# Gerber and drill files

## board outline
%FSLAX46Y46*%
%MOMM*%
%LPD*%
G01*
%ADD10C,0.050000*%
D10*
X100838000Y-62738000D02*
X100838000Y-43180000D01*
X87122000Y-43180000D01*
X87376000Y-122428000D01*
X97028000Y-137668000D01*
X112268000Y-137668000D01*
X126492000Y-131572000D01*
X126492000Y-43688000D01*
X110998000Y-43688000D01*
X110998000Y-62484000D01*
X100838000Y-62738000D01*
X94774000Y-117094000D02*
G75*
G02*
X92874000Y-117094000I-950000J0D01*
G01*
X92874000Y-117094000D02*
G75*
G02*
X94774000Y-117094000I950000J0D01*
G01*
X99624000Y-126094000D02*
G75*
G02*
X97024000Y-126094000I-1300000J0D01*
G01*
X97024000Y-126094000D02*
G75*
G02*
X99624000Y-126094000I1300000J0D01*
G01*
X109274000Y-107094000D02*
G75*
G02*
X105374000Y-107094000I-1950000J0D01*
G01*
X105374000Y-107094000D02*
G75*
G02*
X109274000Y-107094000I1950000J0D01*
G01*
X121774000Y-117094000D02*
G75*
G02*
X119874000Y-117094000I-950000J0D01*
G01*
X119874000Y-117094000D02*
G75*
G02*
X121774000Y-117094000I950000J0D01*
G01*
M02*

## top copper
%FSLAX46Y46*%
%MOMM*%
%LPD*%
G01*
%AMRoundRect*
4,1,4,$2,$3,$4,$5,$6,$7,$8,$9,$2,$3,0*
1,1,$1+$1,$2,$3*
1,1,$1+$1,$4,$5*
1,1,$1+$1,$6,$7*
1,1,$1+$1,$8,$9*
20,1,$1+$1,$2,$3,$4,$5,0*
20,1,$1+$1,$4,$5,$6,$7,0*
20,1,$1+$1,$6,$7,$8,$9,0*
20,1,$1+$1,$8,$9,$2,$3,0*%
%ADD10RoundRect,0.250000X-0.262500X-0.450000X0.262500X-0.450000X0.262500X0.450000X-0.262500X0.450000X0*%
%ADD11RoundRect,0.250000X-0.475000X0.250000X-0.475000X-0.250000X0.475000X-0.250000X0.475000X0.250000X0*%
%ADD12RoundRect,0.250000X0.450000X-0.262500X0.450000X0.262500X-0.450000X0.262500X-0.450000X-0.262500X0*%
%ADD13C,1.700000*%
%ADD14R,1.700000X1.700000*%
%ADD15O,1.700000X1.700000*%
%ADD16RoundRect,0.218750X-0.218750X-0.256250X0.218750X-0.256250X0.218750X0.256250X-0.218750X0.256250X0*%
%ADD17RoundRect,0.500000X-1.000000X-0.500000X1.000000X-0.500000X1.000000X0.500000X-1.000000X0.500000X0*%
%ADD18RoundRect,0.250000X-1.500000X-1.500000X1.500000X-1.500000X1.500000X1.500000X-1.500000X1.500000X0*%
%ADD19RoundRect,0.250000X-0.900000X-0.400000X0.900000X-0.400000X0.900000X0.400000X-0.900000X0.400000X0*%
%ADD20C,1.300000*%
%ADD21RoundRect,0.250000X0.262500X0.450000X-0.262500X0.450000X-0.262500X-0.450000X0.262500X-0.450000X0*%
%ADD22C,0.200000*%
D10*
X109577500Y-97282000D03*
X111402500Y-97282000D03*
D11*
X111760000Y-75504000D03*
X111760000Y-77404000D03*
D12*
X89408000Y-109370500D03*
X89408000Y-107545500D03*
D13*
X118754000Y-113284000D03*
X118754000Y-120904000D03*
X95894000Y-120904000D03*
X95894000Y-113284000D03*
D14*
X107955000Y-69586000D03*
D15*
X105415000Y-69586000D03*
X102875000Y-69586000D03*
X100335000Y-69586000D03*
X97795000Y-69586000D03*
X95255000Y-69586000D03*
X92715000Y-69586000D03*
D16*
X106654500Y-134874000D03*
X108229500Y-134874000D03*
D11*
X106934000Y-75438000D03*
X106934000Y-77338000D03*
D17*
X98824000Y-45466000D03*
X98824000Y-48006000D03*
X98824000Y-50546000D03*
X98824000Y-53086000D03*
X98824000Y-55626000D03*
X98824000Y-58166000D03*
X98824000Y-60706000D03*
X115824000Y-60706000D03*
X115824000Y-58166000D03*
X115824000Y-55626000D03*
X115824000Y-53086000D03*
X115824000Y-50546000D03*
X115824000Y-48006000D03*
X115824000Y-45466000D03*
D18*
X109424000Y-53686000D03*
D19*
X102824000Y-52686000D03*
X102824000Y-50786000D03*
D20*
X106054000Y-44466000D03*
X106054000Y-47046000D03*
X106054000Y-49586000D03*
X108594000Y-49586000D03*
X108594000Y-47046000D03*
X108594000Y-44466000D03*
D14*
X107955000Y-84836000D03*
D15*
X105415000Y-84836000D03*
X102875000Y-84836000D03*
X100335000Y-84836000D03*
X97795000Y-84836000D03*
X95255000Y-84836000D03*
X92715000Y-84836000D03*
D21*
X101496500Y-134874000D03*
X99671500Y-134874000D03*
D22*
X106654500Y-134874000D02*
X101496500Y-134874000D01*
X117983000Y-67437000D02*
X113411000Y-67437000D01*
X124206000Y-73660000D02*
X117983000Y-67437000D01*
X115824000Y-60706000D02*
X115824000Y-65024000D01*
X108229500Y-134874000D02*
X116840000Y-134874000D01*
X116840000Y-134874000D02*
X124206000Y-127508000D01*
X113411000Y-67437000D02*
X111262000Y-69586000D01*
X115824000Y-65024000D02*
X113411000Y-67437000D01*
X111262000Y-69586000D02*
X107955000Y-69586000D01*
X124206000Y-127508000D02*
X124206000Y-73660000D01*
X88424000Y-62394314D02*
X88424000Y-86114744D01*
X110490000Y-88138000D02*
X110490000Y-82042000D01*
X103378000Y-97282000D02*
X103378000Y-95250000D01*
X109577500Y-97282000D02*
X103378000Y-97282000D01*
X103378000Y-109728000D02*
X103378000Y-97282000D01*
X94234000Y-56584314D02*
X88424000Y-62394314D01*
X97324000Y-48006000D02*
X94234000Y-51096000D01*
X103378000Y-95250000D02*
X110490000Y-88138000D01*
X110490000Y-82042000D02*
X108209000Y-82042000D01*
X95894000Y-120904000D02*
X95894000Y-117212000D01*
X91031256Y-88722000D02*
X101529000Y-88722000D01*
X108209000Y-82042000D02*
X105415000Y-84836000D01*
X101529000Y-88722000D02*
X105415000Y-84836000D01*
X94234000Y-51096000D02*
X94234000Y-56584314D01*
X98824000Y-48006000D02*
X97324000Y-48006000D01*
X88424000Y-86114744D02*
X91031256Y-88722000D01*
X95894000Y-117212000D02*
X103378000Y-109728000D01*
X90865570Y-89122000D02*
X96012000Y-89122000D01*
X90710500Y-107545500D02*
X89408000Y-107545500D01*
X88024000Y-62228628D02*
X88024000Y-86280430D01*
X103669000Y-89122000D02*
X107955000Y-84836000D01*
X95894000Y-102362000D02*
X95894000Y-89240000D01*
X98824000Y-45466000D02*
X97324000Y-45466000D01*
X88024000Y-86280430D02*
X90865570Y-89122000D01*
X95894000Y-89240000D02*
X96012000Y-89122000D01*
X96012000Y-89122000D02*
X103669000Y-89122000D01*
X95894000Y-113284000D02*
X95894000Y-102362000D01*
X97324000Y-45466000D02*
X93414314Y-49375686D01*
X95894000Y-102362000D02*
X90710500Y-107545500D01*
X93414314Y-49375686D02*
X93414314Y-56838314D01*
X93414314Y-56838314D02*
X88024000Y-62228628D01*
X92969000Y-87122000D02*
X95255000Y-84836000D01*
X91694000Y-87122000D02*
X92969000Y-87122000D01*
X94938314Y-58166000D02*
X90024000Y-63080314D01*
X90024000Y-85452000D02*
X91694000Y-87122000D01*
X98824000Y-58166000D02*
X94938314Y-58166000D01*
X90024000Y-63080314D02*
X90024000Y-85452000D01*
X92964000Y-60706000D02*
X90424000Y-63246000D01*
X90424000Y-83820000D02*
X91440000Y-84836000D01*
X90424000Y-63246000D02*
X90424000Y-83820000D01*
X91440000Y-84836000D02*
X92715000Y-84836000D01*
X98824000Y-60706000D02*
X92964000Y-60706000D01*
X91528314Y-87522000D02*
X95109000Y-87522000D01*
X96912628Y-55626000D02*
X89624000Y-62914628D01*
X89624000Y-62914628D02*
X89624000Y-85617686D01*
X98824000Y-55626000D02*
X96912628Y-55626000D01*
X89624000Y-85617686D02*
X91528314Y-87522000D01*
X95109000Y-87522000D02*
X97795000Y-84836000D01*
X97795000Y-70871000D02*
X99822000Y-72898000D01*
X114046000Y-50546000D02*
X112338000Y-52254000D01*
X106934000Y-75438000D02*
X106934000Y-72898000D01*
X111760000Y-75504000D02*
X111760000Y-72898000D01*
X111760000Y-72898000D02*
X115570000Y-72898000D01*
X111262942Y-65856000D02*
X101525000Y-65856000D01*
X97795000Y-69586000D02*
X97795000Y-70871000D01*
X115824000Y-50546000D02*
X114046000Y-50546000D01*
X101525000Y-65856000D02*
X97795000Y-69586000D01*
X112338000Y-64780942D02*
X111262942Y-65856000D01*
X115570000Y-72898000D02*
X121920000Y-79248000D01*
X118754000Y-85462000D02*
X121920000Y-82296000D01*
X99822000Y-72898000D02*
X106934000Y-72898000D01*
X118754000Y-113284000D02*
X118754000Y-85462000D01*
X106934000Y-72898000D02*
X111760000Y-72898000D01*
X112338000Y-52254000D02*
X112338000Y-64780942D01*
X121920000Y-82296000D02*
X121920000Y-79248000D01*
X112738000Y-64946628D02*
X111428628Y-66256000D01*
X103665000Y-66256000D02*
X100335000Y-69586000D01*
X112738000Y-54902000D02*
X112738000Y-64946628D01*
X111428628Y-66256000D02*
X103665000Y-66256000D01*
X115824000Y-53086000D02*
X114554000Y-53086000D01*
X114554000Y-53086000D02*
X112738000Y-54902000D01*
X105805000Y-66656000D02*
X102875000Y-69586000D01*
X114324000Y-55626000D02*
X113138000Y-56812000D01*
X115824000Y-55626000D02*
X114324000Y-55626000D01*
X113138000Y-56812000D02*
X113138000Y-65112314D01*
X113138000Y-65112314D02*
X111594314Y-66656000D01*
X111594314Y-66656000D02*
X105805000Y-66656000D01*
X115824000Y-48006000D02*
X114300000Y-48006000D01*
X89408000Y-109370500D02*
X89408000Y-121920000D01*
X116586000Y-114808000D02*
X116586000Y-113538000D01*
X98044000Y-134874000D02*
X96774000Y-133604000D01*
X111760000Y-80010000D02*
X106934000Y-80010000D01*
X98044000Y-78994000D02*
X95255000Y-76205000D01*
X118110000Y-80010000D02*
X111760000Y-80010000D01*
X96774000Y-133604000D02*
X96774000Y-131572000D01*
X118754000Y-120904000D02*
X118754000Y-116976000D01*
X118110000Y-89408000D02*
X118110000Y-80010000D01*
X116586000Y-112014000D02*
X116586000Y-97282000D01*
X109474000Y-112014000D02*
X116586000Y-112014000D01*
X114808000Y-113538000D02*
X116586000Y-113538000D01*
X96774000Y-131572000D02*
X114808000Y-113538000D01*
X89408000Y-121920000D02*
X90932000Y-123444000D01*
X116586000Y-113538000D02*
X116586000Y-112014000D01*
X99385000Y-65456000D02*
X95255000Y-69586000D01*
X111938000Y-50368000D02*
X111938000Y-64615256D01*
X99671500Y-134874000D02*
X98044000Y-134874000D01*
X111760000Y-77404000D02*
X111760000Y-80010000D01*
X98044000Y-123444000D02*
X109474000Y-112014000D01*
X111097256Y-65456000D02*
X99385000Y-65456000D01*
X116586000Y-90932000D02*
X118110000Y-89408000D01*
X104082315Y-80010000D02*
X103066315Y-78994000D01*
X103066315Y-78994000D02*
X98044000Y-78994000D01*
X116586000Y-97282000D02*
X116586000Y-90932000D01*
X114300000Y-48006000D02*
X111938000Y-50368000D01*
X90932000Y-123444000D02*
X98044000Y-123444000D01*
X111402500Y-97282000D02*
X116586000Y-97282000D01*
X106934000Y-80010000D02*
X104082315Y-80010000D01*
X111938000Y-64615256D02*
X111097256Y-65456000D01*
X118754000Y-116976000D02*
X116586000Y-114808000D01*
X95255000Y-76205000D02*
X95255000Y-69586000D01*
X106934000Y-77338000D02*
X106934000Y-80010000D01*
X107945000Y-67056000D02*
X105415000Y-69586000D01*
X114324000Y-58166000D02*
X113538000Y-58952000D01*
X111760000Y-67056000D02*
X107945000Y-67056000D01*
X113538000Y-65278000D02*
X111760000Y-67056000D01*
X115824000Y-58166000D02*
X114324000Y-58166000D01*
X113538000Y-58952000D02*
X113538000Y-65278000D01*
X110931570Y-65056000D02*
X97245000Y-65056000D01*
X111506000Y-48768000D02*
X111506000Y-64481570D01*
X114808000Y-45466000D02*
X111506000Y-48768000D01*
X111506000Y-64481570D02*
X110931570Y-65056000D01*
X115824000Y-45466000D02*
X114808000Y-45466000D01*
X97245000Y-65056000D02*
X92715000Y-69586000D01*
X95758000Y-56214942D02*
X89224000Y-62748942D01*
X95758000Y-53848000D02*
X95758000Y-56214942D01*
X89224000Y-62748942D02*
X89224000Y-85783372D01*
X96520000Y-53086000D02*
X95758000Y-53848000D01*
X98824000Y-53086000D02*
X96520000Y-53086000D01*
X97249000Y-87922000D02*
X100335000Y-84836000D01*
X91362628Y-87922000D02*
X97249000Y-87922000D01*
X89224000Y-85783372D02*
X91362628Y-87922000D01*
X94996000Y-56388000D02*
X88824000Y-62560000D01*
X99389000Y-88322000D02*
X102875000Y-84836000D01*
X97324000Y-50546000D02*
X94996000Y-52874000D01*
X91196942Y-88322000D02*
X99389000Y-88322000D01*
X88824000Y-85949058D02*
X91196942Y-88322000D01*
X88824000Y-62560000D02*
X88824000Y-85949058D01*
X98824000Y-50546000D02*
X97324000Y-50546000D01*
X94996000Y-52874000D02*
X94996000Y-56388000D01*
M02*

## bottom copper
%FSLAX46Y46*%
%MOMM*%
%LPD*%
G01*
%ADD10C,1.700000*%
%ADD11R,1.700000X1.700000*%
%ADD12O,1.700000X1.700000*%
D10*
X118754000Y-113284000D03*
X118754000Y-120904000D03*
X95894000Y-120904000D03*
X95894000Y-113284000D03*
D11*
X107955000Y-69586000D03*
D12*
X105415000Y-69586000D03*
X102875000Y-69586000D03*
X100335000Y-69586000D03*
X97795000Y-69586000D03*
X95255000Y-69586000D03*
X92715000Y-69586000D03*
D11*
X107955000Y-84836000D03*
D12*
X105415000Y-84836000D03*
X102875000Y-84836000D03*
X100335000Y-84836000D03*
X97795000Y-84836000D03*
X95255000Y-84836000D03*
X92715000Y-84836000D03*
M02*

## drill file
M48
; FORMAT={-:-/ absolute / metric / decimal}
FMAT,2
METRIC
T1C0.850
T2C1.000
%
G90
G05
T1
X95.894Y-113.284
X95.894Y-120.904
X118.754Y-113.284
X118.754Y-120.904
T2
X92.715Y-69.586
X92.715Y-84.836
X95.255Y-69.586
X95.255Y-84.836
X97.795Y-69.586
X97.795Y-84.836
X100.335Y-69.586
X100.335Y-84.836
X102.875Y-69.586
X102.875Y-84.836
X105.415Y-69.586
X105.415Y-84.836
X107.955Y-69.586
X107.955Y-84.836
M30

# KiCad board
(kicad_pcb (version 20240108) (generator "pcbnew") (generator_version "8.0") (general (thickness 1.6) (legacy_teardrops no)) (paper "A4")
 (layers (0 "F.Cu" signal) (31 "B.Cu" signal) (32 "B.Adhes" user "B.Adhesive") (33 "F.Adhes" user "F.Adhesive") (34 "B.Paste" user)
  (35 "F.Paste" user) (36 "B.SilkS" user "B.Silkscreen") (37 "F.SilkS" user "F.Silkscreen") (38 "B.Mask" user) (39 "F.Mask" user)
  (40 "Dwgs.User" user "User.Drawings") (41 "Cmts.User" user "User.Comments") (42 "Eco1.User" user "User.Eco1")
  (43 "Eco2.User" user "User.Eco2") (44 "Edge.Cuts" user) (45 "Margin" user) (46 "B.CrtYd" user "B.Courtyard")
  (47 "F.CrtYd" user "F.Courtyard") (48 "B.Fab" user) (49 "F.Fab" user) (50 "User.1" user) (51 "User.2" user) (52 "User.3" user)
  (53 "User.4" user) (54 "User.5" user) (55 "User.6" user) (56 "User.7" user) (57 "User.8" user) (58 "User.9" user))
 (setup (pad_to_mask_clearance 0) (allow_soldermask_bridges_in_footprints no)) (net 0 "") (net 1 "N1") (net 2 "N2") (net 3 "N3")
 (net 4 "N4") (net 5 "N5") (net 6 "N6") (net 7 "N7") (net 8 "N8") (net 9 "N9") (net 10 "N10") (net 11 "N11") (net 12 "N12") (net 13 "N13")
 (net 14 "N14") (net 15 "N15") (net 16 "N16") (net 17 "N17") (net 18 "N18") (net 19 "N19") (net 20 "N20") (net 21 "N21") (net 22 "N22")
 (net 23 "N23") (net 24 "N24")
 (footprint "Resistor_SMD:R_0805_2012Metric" (layer "F.Cu") (at 110.49 97.282)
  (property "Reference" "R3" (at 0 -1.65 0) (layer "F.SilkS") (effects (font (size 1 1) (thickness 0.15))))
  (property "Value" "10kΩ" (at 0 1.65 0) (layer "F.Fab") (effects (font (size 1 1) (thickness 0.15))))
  (pad "1" smd roundrect (at -0.9125 0) (size 1.025 1.4) (layers "F.Cu" "F.Paste" "F.Mask") (roundrect_rratio 0.243902) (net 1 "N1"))
  (pad "2" smd roundrect (at 0.9125 0) (size 1.025 1.4) (layers "F.Cu" "F.Paste" "F.Mask") (roundrect_rratio 0.243902) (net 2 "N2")))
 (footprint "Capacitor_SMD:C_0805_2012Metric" (layer "F.Cu") (at 111.76 76.454 -90)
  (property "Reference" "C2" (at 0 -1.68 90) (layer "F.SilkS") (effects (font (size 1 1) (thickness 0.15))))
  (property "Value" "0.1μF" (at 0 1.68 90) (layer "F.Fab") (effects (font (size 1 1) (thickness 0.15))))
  (pad "1" smd roundrect (at -0.95 0 270) (size 1 1.45) (layers "F.Cu" "F.Paste" "F.Mask") (roundrect_rratio 0.25) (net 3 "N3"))
  (pad "2" smd roundrect (at 0.95 0 270) (size 1 1.45) (layers "F.Cu" "F.Paste" "F.Mask") (roundrect_rratio 0.25) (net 2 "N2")))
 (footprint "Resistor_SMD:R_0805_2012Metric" (layer "F.Cu") (at 89.408 108.458 90)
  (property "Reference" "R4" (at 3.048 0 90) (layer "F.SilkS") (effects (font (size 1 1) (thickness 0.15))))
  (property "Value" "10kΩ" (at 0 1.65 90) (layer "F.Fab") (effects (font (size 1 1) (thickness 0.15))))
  (pad "1" smd roundrect (at -0.9125 0 90) (size 1.025 1.4) (layers "F.Cu" "F.Paste" "F.Mask") (roundrect_rratio 0.243902) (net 2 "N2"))
  (pad "2" smd roundrect (at 0.9125 0 90) (size 1.025 1.4) (layers "F.Cu" "F.Paste" "F.Mask") (roundrect_rratio 0.243902) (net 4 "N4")))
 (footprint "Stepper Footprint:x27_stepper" (layer "F.Cu") (at 109.864 127.254)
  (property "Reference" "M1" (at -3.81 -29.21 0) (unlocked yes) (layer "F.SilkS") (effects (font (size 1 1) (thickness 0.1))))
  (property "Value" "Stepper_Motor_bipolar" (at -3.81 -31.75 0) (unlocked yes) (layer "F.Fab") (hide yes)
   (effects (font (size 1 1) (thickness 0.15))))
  (fp_circle (center -16.04 -10.16) (end -15.09 -10.16) (stroke (width 0.05) (type default)) (fill none) (layer "Edge.Cuts"))
  (fp_circle (center -11.54 -1.16) (end -10.24 -1.16) (stroke (width 0.05) (type default)) (fill none) (layer "Edge.Cuts"))
  (fp_circle (center -2.54 -20.16) (end -0.59 -20.16) (stroke (width 0.05) (type default)) (fill none) (layer "Edge.Cuts"))
  (fp_circle (center 10.96 -10.16) (end 11.91 -10.16) (stroke (width 0.05) (type default)) (fill none) (layer "Edge.Cuts"))
  (pad "1" thru_hole circle (at 8.89 -13.97) (size 1.7 1.7) (drill 0.85) (layers "*.Cu" "*.Mask") (remove_unused_layers no) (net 3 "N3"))
  (pad "2" thru_hole circle (at 8.89 -6.35) (size 1.7 1.7) (drill 0.85) (layers "*.Cu" "*.Mask") (remove_unused_layers no) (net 2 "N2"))
  (pad "3" thru_hole circle (at -13.97 -6.35) (size 1.7 1.7) (drill 0.85) (layers "*.Cu" "*.Mask") (remove_unused_layers no) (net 1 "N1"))
  (pad "4" thru_hole circle (at -13.97 -13.97) (size 1.7 1.7) (drill 0.85) (layers "*.Cu" "*.Mask") (remove_unused_layers no) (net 4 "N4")))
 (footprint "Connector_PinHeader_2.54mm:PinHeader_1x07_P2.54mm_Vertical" (layer "F.Cu") (at 107.955 69.586 -90)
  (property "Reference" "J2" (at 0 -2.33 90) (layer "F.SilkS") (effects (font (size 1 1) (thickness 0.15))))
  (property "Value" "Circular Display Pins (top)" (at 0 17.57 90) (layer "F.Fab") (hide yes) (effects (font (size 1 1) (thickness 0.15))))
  (pad "1" thru_hole rect (at 0 0 270) (size 1.7 1.7) (drill 1) (layers "*.Cu" "*.Mask") (remove_unused_layers no) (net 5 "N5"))
  (pad "2" thru_hole oval (at 0 2.54 270) (size 1.7 1.7) (drill 1) (layers "*.Cu" "*.Mask") (remove_unused_layers no) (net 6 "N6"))
  (pad "3" thru_hole oval (at 0 5.08 270) (size 1.7 1.7) (drill 1) (layers "*.Cu" "*.Mask") (remove_unused_layers no) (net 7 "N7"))
  (pad "4" thru_hole oval (at 0 7.62 270) (size 1.7 1.7) (drill 1) (layers "*.Cu" "*.Mask") (remove_unused_layers no) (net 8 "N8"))
  (pad "5" thru_hole oval (at 0 10.16 270) (size 1.7 1.7) (drill 1) (layers "*.Cu" "*.Mask") (remove_unused_layers no) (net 3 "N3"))
  (pad "6" thru_hole oval (at 0 12.7 270) (size 1.7 1.7) (drill 1) (layers "*.Cu" "*.Mask") (remove_unused_layers no) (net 2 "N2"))
  (pad "7" thru_hole oval (at 0 15.24 270) (size 1.7 1.7) (drill 1) (layers "*.Cu" "*.Mask") (remove_unused_layers no) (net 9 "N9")))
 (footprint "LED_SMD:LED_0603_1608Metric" (layer "F.Cu") (at 107.442 134.874)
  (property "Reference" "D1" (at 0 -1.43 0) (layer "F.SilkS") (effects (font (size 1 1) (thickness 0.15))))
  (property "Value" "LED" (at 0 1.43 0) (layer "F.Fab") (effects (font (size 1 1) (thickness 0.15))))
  (pad "1" smd roundrect (at -0.7875 0) (size 0.875 0.95) (layers "F.Cu" "F.Paste" "F.Mask") (roundrect_rratio 0.25) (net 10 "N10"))
  (pad "2" smd roundrect (at 0.7875 0) (size 0.875 0.95) (layers "F.Cu" "F.Paste" "F.Mask") (roundrect_rratio 0.25) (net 5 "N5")))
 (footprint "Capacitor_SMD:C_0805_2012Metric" (layer "F.Cu") (at 106.934 76.388 -90)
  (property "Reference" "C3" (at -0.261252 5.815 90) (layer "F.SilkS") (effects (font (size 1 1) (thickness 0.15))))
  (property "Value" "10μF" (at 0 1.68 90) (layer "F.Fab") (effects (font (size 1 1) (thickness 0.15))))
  (pad "1" smd roundrect (at -0.95 0 270) (size 1 1.45) (layers "F.Cu" "F.Paste" "F.Mask") (roundrect_rratio 0.25) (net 3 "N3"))
  (pad "2" smd roundrect (at 0.95 0 270) (size 1 1.45) (layers "F.Cu" "F.Paste" "F.Mask") (roundrect_rratio 0.25) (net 2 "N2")))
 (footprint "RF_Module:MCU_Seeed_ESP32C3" (layer "F.Cu") (at 107.324 53.086)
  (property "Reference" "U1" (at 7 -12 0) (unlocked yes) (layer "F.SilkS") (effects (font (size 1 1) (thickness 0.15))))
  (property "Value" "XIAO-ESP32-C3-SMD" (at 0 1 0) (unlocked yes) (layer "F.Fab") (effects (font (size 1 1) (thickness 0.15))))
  (pad "" smd roundrect (at 1.1 -0.4) (size 1.5 1.5) (layers "F.Paste") (roundrect_rratio 0.1666666667))
  (pad "" smd roundrect (at 1.1 1.6) (size 1.5 1.5) (layers "F.Paste") (roundrect_rratio 0.1666666667))
  (pad "" smd roundrect (at 3.1 -0.4) (size 1.5 1.5) (layers "F.Paste") (roundrect_rratio 0.1666666667))
  (pad "" smd roundrect (at 3.1 1.6) (size 1.5 1.5) (layers "F.Paste") (roundrect_rratio 0.1666666667))
  (pad "1" smd roundrect (at -8.5 -7.62) (size 3 2) (layers "F.Cu" "F.Paste" "F.Mask") (roundrect_rratio 0.25) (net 4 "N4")
   (thermal_bridge_angle 45))
  (pad "2" smd roundrect (at -8.5 -5.08) (size 3 2) (layers "F.Cu" "F.Paste" "F.Mask") (roundrect_rratio 0.25) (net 1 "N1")
   (thermal_bridge_angle 45))
  (pad "3" smd roundrect (at -8.5 -2.54) (size 3 2) (layers "F.Cu" "F.Paste" "F.Mask") (roundrect_rratio 0.25) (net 5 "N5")
   (thermal_bridge_angle 45))
  (pad "4" smd roundrect (at -8.5 0) (size 3 2) (layers "F.Cu" "F.Paste" "F.Mask") (roundrect_rratio 0.25) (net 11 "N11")
   (thermal_bridge_angle 45))
  (pad "5" smd roundrect (at -8.5 2.54) (size 3 2) (layers "F.Cu" "F.Paste" "F.Mask") (roundrect_rratio 0.25) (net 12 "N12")
   (thermal_bridge_angle 45))
  (pad "6" smd roundrect (at -8.5 5.08) (size 3 2) (layers "F.Cu" "F.Paste" "F.Mask") (roundrect_rratio 0.25) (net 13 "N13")
   (thermal_bridge_angle 45))
  (pad "7" smd roundrect (at -8.5 7.62) (size 3 2) (layers "F.Cu" "F.Paste" "F.Mask") (roundrect_rratio 0.25) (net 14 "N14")
   (thermal_bridge_angle 45))
  (pad "8" smd roundrect (at 8.5 7.62) (size 3 2) (layers "F.Cu" "F.Paste" "F.Mask") (roundrect_rratio 0.25) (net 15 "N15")
   (thermal_bridge_angle 45))
  (pad "9" smd roundrect (at 8.5 5.08) (size 3 2) (layers "F.Cu" "F.Paste" "F.Mask") (roundrect_rratio 0.25) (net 6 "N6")
   (thermal_bridge_angle 45))
  (pad "10" smd roundrect (at 8.5 2.54) (size 3 2) (layers "F.Cu" "F.Paste" "F.Mask") (roundrect_rratio 0.25) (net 7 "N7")
   (thermal_bridge_angle 45))
  (pad "11" smd roundrect (at 8.5 0) (size 3 2) (layers "F.Cu" "F.Paste" "F.Mask") (roundrect_rratio 0.25) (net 8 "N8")
   (thermal_bridge_angle 45))
  (pad "12" smd roundrect (at 8.5 -2.54) (size 3 2) (layers "F.Cu" "F.Paste" "F.Mask") (roundrect_rratio 0.25) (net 3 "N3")
   (thermal_bridge_angle 45))
  (pad "13" smd roundrect (at 8.5 -5.08) (size 3 2) (layers "F.Cu" "F.Paste" "F.Mask") (roundrect_rratio 0.25) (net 2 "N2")
   (thermal_bridge_angle 45))
  (pad "14" smd roundrect (at 8.5 -7.62) (size 3 2) (layers "F.Cu" "F.Paste" "F.Mask") (roundrect_rratio 0.25) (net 9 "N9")
   (thermal_bridge_angle 45))
  (pad "15" smd roundrect (at 2.1 0.6) (size 3.5 3.5) (layers "F.Cu" "F.Mask") (roundrect_rratio 0.07142857143) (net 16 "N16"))
  (pad "16" smd roundrect (at -4.5 -0.4) (size 2.3 1.3) (layers "F.Cu" "F.Paste" "F.Mask") (roundrect_rratio 0.1923076923) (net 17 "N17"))
  (pad "17" smd roundrect (at -4.5 -2.3) (size 2.3 1.3) (layers "F.Cu" "F.Paste" "F.Mask") (roundrect_rratio 0.1923076923) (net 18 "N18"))
  (pad "18" smd circle (at -1.27 -8.62) (size 1.3 1.3) (layers "F.Cu" "F.Paste" "F.Mask") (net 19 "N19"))
  (pad "19" smd circle (at -1.27 -6.04) (size 1.3 1.3) (layers "F.Cu" "F.Paste" "F.Mask") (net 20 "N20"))
  (pad "20" smd circle (at -1.27 -3.5) (size 1.3 1.3) (layers "F.Cu" "F.Paste" "F.Mask") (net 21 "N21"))
  (pad "21" smd circle (at 1.27 -3.5) (size 1.3 1.3) (layers "F.Cu" "F.Paste" "F.Mask") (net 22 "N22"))
  (pad "22" smd circle (at 1.27 -6.04) (size 1.3 1.3) (layers "F.Cu" "F.Paste" "F.Mask") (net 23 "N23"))
  (pad "23" smd circle (at 1.27 -8.62) (size 1.3 1.3) (layers "F.Cu" "F.Paste" "F.Mask")))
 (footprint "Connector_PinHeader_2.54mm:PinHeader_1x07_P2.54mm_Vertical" (layer "F.Cu") (at 107.955 84.836 -90)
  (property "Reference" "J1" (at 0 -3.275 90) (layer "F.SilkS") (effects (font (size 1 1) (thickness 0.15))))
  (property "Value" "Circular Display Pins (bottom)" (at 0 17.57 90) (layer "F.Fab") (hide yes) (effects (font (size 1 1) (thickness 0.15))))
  (pad "1" thru_hole rect (at 0 0 270) (size 1.7 1.7) (drill 1) (layers "*.Cu" "*.Mask") (remove_unused_layers no) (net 4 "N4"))
  (pad "2" thru_hole oval (at 0 2.54 270) (size 1.7 1.7) (drill 1) (layers "*.Cu" "*.Mask") (remove_unused_layers no) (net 1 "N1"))
  (pad "3" thru_hole oval (at 0 5.08 270) (size 1.7 1.7) (drill 1) (layers "*.Cu" "*.Mask") (remove_unused_layers no) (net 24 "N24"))
  (pad "4" thru_hole oval (at 0 7.62 270) (size 1.7 1.7) (drill 1) (layers "*.Cu" "*.Mask") (remove_unused_layers no) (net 11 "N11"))
  (pad "5" thru_hole oval (at 0 10.16 270) (size 1.7 1.7) (drill 1) (layers "*.Cu" "*.Mask") (remove_unused_layers no) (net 12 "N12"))
  (pad "6" thru_hole oval (at 0 12.7 270) (size 1.7 1.7) (drill 1) (layers "*.Cu" "*.Mask") (remove_unused_layers no) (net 13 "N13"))
  (pad "7" thru_hole oval (at 0 15.24 270) (size 1.7 1.7) (drill 1) (layers "*.Cu" "*.Mask") (remove_unused_layers no) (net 14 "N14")))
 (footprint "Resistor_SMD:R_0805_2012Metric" (layer "F.Cu") (at 100.584 134.874 180)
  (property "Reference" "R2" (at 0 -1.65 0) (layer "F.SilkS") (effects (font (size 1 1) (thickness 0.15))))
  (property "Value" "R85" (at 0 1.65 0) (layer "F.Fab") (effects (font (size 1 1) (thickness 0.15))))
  (pad "1" smd roundrect (at -0.9125 0 180) (size 1.025 1.4) (layers "F.Cu" "F.Paste" "F.Mask") (roundrect_rratio 0.243902) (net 10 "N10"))
  (pad "2" smd roundrect (at 0.9125 0 180) (size 1.025 1.4) (layers "F.Cu" "F.Paste" "F.Mask") (roundrect_rratio 0.243902) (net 2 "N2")))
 (gr_poly
  (pts (xy 100.838 62.738) (xy 100.838 43.18) (xy 87.122 43.18) (xy 87.376 122.428) (xy 97.028 137.668) (xy 112.268 137.668)
   (xy 126.492 131.572) (xy 126.492 43.688) (xy 110.998 43.688) (xy 110.998 62.484))
  (stroke (width 0.05) (type solid)) (fill none) (layer "Edge.Cuts"))
 (segment (start 106.6545 134.874) (end 101.4965 134.874) (width 0.2) (layer "F.Cu") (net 10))
 (segment (start 117.983 67.437) (end 113.411 67.437) (width 0.2) (layer "F.Cu") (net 5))
 (segment (start 124.206 73.66) (end 117.983 67.437) (width 0.2) (layer "F.Cu") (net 5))
 (segment (start 115.824 60.706) (end 115.824 65.024) (width 0.2) (layer "F.Cu") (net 5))
 (segment (start 108.2295 134.874) (end 116.84 134.874) (width 0.2) (layer "F.Cu") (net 5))
 (segment (start 116.84 134.874) (end 124.206 127.508) (width 0.2) (layer "F.Cu") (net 5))
 (segment (start 113.411 67.437) (end 111.262 69.586) (width 0.2) (layer "F.Cu") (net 5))
 (segment (start 115.824 65.024) (end 113.411 67.437) (width 0.2) (layer "F.Cu") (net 5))
 (segment (start 111.262 69.586) (end 107.955 69.586) (width 0.2) (layer "F.Cu") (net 5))
 (segment (start 124.206 127.508) (end 124.206 73.66) (width 0.2) (layer "F.Cu") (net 5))
 (segment (start 88.424 62.394314) (end 88.424 86.114744) (width 0.2) (layer "F.Cu") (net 1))
 (segment (start 110.49 88.138) (end 110.49 82.042) (width 0.2) (layer "F.Cu") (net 1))
 (segment (start 103.378 97.282) (end 103.378 95.25) (width 0.2) (layer "F.Cu") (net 1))
 (segment (start 109.5775 97.282) (end 103.378 97.282) (width 0.2) (layer "F.Cu") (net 1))
 (segment (start 103.378 109.728) (end 103.378 97.282) (width 0.2) (layer "F.Cu") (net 1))
 (segment (start 94.234 56.584314) (end 88.424 62.394314) (width 0.2) (layer "F.Cu") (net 1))
 (segment (start 97.324 48.006) (end 94.234 51.096) (width 0.2) (layer "F.Cu") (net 1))
 (segment (start 103.378 95.25) (end 110.49 88.138) (width 0.2) (layer "F.Cu") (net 1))
 (segment (start 110.49 82.042) (end 108.209 82.042) (width 0.2) (layer "F.Cu") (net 1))
 (segment (start 95.894 120.904) (end 95.894 117.212) (width 0.2) (layer "F.Cu") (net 1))
 (segment (start 91.031256 88.722) (end 101.529 88.722) (width 0.2) (layer "F.Cu") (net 1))
 (segment (start 108.209 82.042) (end 105.415 84.836) (width 0.2) (layer "F.Cu") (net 1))
 (segment (start 101.529 88.722) (end 105.415 84.836) (width 0.2) (layer "F.Cu") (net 1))
 (segment (start 94.234 51.096) (end 94.234 56.584314) (width 0.2) (layer "F.Cu") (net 1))
 (segment (start 98.824 48.006) (end 97.324 48.006) (width 0.2) (layer "F.Cu") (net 1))
 (segment (start 88.424 86.114744) (end 91.031256 88.722) (width 0.2) (layer "F.Cu") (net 1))
 (segment (start 95.894 117.212) (end 103.378 109.728) (width 0.2) (layer "F.Cu") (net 1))
 (segment (start 90.86557 89.122) (end 96.012 89.122) (width 0.2) (layer "F.Cu") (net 4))
 (segment (start 90.7105 107.5455) (end 89.408 107.5455) (width 0.2) (layer "F.Cu") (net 4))
 (segment (start 88.024 62.228628) (end 88.024 86.28043) (width 0.2) (layer "F.Cu") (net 4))
 (segment (start 103.669 89.122) (end 107.955 84.836) (width 0.2) (layer "F.Cu") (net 4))
 (segment (start 95.894 102.362) (end 95.894 89.24) (width 0.2) (layer "F.Cu") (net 4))
 (segment (start 98.824 45.466) (end 97.324 45.466) (width 0.2) (layer "F.Cu") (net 4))
 (segment (start 88.024 86.28043) (end 90.86557 89.122) (width 0.2) (layer "F.Cu") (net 4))
 (segment (start 95.894 89.24) (end 96.012 89.122) (width 0.2) (layer "F.Cu") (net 4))
 (segment (start 96.012 89.122) (end 103.669 89.122) (width 0.2) (layer "F.Cu") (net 4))
 (segment (start 95.894 113.284) (end 95.894 102.362) (width 0.2) (layer "F.Cu") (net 4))
 (segment (start 97.324 45.466) (end 93.414314 49.375686) (width 0.2) (layer "F.Cu") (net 4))
 (segment (start 95.894 102.362) (end 90.7105 107.5455) (width 0.2) (layer "F.Cu") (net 4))
 (segment (start 93.414314 49.375686) (end 93.414314 56.838314) (width 0.2) (layer "F.Cu") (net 4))
 (segment (start 93.414314 56.838314) (end 88.024 62.228628) (width 0.2) (layer "F.Cu") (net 4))
 (segment (start 92.969 87.122) (end 95.255 84.836) (width 0.2) (layer "F.Cu") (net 13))
 (segment (start 91.694 87.122) (end 92.969 87.122) (width 0.2) (layer "F.Cu") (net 13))
 (segment (start 94.938314 58.166) (end 90.024 63.080314) (width 0.2) (layer "F.Cu") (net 13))
 (segment (start 90.024 85.452) (end 91.694 87.122) (width 0.2) (layer "F.Cu") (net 13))
 (segment (start 98.824 58.166) (end 94.938314 58.166) (width 0.2) (layer "F.Cu") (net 13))
 (segment (start 90.024 63.080314) (end 90.024 85.452) (width 0.2) (layer "F.Cu") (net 13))
 (segment (start 92.964 60.706) (end 90.424 63.246) (width 0.2) (layer "F.Cu") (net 14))
 (segment (start 90.424 83.82) (end 91.44 84.836) (width 0.2) (layer "F.Cu") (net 14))
 (segment (start 90.424 63.246) (end 90.424 83.82) (width 0.2) (layer "F.Cu") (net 14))
 (segment (start 91.44 84.836) (end 92.715 84.836) (width 0.2) (layer "F.Cu") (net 14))
 (segment (start 98.824 60.706) (end 92.964 60.706) (width 0.2) (layer "F.Cu") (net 14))
 (segment (start 91.528314 87.522) (end 95.109 87.522) (width 0.2) (layer "F.Cu") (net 12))
 (segment (start 96.912628 55.626) (end 89.624 62.914628) (width 0.2) (layer "F.Cu") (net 12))
 (segment (start 89.624 62.914628) (end 89.624 85.617686) (width 0.2) (layer "F.Cu") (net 12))
 (segment (start 98.824 55.626) (end 96.912628 55.626) (width 0.2) (layer "F.Cu") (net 12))
 (segment (start 89.624 85.617686) (end 91.528314 87.522) (width 0.2) (layer "F.Cu") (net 12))
 (segment (start 95.109 87.522) (end 97.795 84.836) (width 0.2) (layer "F.Cu") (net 12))
 (segment (start 97.795 70.871) (end 99.822 72.898) (width 0.2) (layer "F.Cu") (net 3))
 (segment (start 114.046 50.546) (end 112.338 52.254) (width 0.2) (layer "F.Cu") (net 3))
 (segment (start 106.934 75.438) (end 106.934 72.898) (width 0.2) (layer "F.Cu") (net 3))
 (segment (start 111.76 75.504) (end 111.76 72.898) (width 0.2) (layer "F.Cu") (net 3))
 (segment (start 111.76 72.898) (end 115.57 72.898) (width 0.2) (layer "F.Cu") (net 3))
 (segment (start 111.262942 65.856) (end 101.525 65.856) (width 0.2) (layer "F.Cu") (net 3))
 (segment (start 97.795 69.586) (end 97.795 70.871) (width 0.2) (layer "F.Cu") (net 3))
 (segment (start 115.824 50.546) (end 114.046 50.546) (width 0.2) (layer "F.Cu") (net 3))
 (segment (start 101.525 65.856) (end 97.795 69.586) (width 0.2) (layer "F.Cu") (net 3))
 (segment (start 112.338 64.780942) (end 111.262942 65.856) (width 0.2) (layer "F.Cu") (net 3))
 (segment (start 115.57 72.898) (end 121.92 79.248) (width 0.2) (layer "F.Cu") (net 3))
 (segment (start 118.754 85.462) (end 121.92 82.296) (width 0.2) (layer "F.Cu") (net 3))
 (segment (start 99.822 72.898) (end 106.934 72.898) (width 0.2) (layer "F.Cu") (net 3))
 (segment (start 118.754 113.284) (end 118.754 85.462) (width 0.2) (layer "F.Cu") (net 3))
 (segment (start 106.934 72.898) (end 111.76 72.898) (width 0.2) (layer "F.Cu") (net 3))
 (segment (start 112.338 52.254) (end 112.338 64.780942) (width 0.2) (layer "F.Cu") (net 3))
 (segment (start 121.92 82.296) (end 121.92 79.248) (width 0.2) (layer "F.Cu") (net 3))
 (segment (start 112.738 64.946628) (end 111.428628 66.256) (width 0.2) (layer "F.Cu") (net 8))
 (segment (start 103.665 66.256) (end 100.335 69.586) (width 0.2) (layer "F.Cu") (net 8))
 (segment (start 112.738 54.902) (end 112.738 64.946628) (width 0.2) (layer "F.Cu") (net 8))
 (segment (start 111.428628 66.256) (end 103.665 66.256) (width 0.2) (layer "F.Cu") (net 8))
 (segment (start 115.824 53.086) (end 114.554 53.086) (width 0.2) (layer "F.Cu") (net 8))
 (segment (start 114.554 53.086) (end 112.738 54.902) (width 0.2) (layer "F.Cu") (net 8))
 (segment (start 105.805 66.656) (end 102.875 69.586) (width 0.2) (layer "F.Cu") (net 7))
 (segment (start 114.324 55.626) (end 113.138 56.812) (width 0.2) (layer "F.Cu") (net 7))
 (segment (start 115.824 55.626) (end 114.324 55.626) (width 0.2) (layer "F.Cu") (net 7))
 (segment (start 113.138 56.812) (end 113.138 65.112314) (width 0.2) (layer "F.Cu") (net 7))
 (segment (start 113.138 65.112314) (end 111.594314 66.656) (width 0.2) (layer "F.Cu") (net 7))
 (segment (start 111.594314 66.656) (end 105.805 66.656) (width 0.2) (layer "F.Cu") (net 7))
 (segment (start 115.824 48.006) (end 114.3 48.006) (width 0.2) (layer "F.Cu") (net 2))
 (segment (start 89.408 109.3705) (end 89.408 121.92) (width 0.2) (layer "F.Cu") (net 2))
 (segment (start 116.586 114.808) (end 116.586 113.538) (width 0.2) (layer "F.Cu") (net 2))
 (segment (start 98.044 134.874) (end 96.774 133.604) (width 0.2) (layer "F.Cu") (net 2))
 (segment (start 111.76 80.01) (end 106.934 80.01) (width 0.2) (layer "F.Cu") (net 2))
 (segment (start 98.044 78.994) (end 95.255 76.205) (width 0.2) (layer "F.Cu") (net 2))
 (segment (start 118.11 80.01) (end 111.76 80.01) (width 0.2) (layer "F.Cu") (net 2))
 (segment (start 96.774 133.604) (end 96.774 131.572) (width 0.2) (layer "F.Cu") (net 2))
 (segment (start 118.754 120.904) (end 118.754 116.976) (width 0.2) (layer "F.Cu") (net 2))
 (segment (start 118.11 89.408) (end 118.11 80.01) (width 0.2) (layer "F.Cu") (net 2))
 (segment (start 116.586 112.014) (end 116.586 97.282) (width 0.2) (layer "F.Cu") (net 2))
 (segment (start 109.474 112.014) (end 116.586 112.014) (width 0.2) (layer "F.Cu") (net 2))
 (segment (start 114.808 113.538) (end 116.586 113.538) (width 0.2) (layer "F.Cu") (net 2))
 (segment (start 96.774 131.572) (end 114.808 113.538) (width 0.2) (layer "F.Cu") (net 2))
 (segment (start 89.408 121.92) (end 90.932 123.444) (width 0.2) (layer "F.Cu") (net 2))
 (segment (start 116.586 113.538) (end 116.586 112.014) (width 0.2) (layer "F.Cu") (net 2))
 (segment (start 99.385 65.456) (end 95.255 69.586) (width 0.2) (layer "F.Cu") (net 2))
 (segment (start 111.938 50.368) (end 111.938 64.615256) (width 0.2) (layer "F.Cu") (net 2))
 (segment (start 99.6715 134.874) (end 98.044 134.874) (width 0.2) (layer "F.Cu") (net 2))
 (segment (start 111.76 77.404) (end 111.76 80.01) (width 0.2) (layer "F.Cu") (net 2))
 (segment (start 98.044 123.444) (end 109.474 112.014) (width 0.2) (layer "F.Cu") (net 2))
 (segment (start 111.097256 65.456) (end 99.385 65.456) (width 0.2) (layer "F.Cu") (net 2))
 (segment (start 116.586 90.932) (end 118.11 89.408) (width 0.2) (layer "F.Cu") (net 2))
 (segment (start 104.082315 80.01) (end 103.066315 78.994) (width 0.2) (layer "F.Cu") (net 2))
 (segment (start 103.066315 78.994) (end 98.044 78.994) (width 0.2) (layer "F.Cu") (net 2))
 (segment (start 116.586 97.282) (end 116.586 90.932) (width 0.2) (layer "F.Cu") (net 2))
 (segment (start 114.3 48.006) (end 111.938 50.368) (width 0.2) (layer "F.Cu") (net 2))
 (segment (start 90.932 123.444) (end 98.044 123.444) (width 0.2) (layer "F.Cu") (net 2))
 (segment (start 111.4025 97.282) (end 116.586 97.282) (width 0.2) (layer "F.Cu") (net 2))
 (segment (start 106.934 80.01) (end 104.082315 80.01) (width 0.2) (layer "F.Cu") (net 2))
 (segment (start 111.938 64.615256) (end 111.097256 65.456) (width 0.2) (layer "F.Cu") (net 2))
 (segment (start 118.754 116.976) (end 116.586 114.808) (width 0.2) (layer "F.Cu") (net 2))
 (segment (start 95.255 76.205) (end 95.255 69.586) (width 0.2) (layer "F.Cu") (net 2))
 (segment (start 106.934 77.338) (end 106.934 80.01) (width 0.2) (layer "F.Cu") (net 2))
 (segment (start 107.945 67.056) (end 105.415 69.586) (width 0.2) (layer "F.Cu") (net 6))
 (segment (start 114.324 58.166) (end 113.538 58.952) (width 0.2) (layer "F.Cu") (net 6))
 (segment (start 111.76 67.056) (end 107.945 67.056) (width 0.2) (layer "F.Cu") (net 6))
 (segment (start 113.538 65.278) (end 111.76 67.056) (width 0.2) (layer "F.Cu") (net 6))
 (segment (start 115.824 58.166) (end 114.324 58.166) (width 0.2) (layer "F.Cu") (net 6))
 (segment (start 113.538 58.952) (end 113.538 65.278) (width 0.2) (layer "F.Cu") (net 6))
 (segment (start 110.93157 65.056) (end 97.245 65.056) (width 0.2) (layer "F.Cu") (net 9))
 (segment (start 111.506 48.768) (end 111.506 64.48157) (width 0.2) (layer "F.Cu") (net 9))
 (segment (start 114.808 45.466) (end 111.506 48.768) (width 0.2) (layer "F.Cu") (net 9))
 (segment (start 111.506 64.48157) (end 110.93157 65.056) (width 0.2) (layer "F.Cu") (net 9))
 (segment (start 115.824 45.466) (end 114.808 45.466) (width 0.2) (layer "F.Cu") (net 9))
 (segment (start 97.245 65.056) (end 92.715 69.586) (width 0.2) (layer "F.Cu") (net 9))
 (segment (start 95.758 56.214942) (end 89.224 62.748942) (width 0.2) (layer "F.Cu") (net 11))
 (segment (start 95.758 53.848) (end 95.758 56.214942) (width 0.2) (layer "F.Cu") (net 11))
 (segment (start 89.224 62.748942) (end 89.224 85.783372) (width 0.2) (layer "F.Cu") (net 11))
 (segment (start 96.52 53.086) (end 95.758 53.848) (width 0.2) (layer "F.Cu") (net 11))
 (segment (start 98.824 53.086) (end 96.52 53.086) (width 0.2) (layer "F.Cu") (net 11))
 (segment (start 97.249 87.922) (end 100.335 84.836) (width 0.2) (layer "F.Cu") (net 11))
 (segment (start 91.362628 87.922) (end 97.249 87.922) (width 0.2) (layer "F.Cu") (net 11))
 (segment (start 89.224 85.783372) (end 91.362628 87.922) (width 0.2) (layer "F.Cu") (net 11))
 (segment (start 94.996 56.388) (end 88.824 62.56) (width 0.2) (layer "F.Cu") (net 24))
 (segment (start 99.389 88.322) (end 102.875 84.836) (width 0.2) (layer "F.Cu") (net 24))
 (segment (start 97.324 50.546) (end 94.996 52.874) (width 0.2) (layer "F.Cu") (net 24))
 (segment (start 91.196942 88.322) (end 99.389 88.322) (width 0.2) (layer "F.Cu") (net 24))
 (segment (start 88.824 85.949058) (end 91.196942 88.322) (width 0.2) (layer "F.Cu") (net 24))
 (segment (start 88.824 62.56) (end 88.824 85.949058) (width 0.2) (layer "F.Cu") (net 24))
 (segment (start 98.824 50.546) (end 97.324 50.546) (width 0.2) (layer "F.Cu") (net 24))
 (segment (start 94.996 52.874) (end 94.996 56.388) (width 0.2) (layer "F.Cu") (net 24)))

